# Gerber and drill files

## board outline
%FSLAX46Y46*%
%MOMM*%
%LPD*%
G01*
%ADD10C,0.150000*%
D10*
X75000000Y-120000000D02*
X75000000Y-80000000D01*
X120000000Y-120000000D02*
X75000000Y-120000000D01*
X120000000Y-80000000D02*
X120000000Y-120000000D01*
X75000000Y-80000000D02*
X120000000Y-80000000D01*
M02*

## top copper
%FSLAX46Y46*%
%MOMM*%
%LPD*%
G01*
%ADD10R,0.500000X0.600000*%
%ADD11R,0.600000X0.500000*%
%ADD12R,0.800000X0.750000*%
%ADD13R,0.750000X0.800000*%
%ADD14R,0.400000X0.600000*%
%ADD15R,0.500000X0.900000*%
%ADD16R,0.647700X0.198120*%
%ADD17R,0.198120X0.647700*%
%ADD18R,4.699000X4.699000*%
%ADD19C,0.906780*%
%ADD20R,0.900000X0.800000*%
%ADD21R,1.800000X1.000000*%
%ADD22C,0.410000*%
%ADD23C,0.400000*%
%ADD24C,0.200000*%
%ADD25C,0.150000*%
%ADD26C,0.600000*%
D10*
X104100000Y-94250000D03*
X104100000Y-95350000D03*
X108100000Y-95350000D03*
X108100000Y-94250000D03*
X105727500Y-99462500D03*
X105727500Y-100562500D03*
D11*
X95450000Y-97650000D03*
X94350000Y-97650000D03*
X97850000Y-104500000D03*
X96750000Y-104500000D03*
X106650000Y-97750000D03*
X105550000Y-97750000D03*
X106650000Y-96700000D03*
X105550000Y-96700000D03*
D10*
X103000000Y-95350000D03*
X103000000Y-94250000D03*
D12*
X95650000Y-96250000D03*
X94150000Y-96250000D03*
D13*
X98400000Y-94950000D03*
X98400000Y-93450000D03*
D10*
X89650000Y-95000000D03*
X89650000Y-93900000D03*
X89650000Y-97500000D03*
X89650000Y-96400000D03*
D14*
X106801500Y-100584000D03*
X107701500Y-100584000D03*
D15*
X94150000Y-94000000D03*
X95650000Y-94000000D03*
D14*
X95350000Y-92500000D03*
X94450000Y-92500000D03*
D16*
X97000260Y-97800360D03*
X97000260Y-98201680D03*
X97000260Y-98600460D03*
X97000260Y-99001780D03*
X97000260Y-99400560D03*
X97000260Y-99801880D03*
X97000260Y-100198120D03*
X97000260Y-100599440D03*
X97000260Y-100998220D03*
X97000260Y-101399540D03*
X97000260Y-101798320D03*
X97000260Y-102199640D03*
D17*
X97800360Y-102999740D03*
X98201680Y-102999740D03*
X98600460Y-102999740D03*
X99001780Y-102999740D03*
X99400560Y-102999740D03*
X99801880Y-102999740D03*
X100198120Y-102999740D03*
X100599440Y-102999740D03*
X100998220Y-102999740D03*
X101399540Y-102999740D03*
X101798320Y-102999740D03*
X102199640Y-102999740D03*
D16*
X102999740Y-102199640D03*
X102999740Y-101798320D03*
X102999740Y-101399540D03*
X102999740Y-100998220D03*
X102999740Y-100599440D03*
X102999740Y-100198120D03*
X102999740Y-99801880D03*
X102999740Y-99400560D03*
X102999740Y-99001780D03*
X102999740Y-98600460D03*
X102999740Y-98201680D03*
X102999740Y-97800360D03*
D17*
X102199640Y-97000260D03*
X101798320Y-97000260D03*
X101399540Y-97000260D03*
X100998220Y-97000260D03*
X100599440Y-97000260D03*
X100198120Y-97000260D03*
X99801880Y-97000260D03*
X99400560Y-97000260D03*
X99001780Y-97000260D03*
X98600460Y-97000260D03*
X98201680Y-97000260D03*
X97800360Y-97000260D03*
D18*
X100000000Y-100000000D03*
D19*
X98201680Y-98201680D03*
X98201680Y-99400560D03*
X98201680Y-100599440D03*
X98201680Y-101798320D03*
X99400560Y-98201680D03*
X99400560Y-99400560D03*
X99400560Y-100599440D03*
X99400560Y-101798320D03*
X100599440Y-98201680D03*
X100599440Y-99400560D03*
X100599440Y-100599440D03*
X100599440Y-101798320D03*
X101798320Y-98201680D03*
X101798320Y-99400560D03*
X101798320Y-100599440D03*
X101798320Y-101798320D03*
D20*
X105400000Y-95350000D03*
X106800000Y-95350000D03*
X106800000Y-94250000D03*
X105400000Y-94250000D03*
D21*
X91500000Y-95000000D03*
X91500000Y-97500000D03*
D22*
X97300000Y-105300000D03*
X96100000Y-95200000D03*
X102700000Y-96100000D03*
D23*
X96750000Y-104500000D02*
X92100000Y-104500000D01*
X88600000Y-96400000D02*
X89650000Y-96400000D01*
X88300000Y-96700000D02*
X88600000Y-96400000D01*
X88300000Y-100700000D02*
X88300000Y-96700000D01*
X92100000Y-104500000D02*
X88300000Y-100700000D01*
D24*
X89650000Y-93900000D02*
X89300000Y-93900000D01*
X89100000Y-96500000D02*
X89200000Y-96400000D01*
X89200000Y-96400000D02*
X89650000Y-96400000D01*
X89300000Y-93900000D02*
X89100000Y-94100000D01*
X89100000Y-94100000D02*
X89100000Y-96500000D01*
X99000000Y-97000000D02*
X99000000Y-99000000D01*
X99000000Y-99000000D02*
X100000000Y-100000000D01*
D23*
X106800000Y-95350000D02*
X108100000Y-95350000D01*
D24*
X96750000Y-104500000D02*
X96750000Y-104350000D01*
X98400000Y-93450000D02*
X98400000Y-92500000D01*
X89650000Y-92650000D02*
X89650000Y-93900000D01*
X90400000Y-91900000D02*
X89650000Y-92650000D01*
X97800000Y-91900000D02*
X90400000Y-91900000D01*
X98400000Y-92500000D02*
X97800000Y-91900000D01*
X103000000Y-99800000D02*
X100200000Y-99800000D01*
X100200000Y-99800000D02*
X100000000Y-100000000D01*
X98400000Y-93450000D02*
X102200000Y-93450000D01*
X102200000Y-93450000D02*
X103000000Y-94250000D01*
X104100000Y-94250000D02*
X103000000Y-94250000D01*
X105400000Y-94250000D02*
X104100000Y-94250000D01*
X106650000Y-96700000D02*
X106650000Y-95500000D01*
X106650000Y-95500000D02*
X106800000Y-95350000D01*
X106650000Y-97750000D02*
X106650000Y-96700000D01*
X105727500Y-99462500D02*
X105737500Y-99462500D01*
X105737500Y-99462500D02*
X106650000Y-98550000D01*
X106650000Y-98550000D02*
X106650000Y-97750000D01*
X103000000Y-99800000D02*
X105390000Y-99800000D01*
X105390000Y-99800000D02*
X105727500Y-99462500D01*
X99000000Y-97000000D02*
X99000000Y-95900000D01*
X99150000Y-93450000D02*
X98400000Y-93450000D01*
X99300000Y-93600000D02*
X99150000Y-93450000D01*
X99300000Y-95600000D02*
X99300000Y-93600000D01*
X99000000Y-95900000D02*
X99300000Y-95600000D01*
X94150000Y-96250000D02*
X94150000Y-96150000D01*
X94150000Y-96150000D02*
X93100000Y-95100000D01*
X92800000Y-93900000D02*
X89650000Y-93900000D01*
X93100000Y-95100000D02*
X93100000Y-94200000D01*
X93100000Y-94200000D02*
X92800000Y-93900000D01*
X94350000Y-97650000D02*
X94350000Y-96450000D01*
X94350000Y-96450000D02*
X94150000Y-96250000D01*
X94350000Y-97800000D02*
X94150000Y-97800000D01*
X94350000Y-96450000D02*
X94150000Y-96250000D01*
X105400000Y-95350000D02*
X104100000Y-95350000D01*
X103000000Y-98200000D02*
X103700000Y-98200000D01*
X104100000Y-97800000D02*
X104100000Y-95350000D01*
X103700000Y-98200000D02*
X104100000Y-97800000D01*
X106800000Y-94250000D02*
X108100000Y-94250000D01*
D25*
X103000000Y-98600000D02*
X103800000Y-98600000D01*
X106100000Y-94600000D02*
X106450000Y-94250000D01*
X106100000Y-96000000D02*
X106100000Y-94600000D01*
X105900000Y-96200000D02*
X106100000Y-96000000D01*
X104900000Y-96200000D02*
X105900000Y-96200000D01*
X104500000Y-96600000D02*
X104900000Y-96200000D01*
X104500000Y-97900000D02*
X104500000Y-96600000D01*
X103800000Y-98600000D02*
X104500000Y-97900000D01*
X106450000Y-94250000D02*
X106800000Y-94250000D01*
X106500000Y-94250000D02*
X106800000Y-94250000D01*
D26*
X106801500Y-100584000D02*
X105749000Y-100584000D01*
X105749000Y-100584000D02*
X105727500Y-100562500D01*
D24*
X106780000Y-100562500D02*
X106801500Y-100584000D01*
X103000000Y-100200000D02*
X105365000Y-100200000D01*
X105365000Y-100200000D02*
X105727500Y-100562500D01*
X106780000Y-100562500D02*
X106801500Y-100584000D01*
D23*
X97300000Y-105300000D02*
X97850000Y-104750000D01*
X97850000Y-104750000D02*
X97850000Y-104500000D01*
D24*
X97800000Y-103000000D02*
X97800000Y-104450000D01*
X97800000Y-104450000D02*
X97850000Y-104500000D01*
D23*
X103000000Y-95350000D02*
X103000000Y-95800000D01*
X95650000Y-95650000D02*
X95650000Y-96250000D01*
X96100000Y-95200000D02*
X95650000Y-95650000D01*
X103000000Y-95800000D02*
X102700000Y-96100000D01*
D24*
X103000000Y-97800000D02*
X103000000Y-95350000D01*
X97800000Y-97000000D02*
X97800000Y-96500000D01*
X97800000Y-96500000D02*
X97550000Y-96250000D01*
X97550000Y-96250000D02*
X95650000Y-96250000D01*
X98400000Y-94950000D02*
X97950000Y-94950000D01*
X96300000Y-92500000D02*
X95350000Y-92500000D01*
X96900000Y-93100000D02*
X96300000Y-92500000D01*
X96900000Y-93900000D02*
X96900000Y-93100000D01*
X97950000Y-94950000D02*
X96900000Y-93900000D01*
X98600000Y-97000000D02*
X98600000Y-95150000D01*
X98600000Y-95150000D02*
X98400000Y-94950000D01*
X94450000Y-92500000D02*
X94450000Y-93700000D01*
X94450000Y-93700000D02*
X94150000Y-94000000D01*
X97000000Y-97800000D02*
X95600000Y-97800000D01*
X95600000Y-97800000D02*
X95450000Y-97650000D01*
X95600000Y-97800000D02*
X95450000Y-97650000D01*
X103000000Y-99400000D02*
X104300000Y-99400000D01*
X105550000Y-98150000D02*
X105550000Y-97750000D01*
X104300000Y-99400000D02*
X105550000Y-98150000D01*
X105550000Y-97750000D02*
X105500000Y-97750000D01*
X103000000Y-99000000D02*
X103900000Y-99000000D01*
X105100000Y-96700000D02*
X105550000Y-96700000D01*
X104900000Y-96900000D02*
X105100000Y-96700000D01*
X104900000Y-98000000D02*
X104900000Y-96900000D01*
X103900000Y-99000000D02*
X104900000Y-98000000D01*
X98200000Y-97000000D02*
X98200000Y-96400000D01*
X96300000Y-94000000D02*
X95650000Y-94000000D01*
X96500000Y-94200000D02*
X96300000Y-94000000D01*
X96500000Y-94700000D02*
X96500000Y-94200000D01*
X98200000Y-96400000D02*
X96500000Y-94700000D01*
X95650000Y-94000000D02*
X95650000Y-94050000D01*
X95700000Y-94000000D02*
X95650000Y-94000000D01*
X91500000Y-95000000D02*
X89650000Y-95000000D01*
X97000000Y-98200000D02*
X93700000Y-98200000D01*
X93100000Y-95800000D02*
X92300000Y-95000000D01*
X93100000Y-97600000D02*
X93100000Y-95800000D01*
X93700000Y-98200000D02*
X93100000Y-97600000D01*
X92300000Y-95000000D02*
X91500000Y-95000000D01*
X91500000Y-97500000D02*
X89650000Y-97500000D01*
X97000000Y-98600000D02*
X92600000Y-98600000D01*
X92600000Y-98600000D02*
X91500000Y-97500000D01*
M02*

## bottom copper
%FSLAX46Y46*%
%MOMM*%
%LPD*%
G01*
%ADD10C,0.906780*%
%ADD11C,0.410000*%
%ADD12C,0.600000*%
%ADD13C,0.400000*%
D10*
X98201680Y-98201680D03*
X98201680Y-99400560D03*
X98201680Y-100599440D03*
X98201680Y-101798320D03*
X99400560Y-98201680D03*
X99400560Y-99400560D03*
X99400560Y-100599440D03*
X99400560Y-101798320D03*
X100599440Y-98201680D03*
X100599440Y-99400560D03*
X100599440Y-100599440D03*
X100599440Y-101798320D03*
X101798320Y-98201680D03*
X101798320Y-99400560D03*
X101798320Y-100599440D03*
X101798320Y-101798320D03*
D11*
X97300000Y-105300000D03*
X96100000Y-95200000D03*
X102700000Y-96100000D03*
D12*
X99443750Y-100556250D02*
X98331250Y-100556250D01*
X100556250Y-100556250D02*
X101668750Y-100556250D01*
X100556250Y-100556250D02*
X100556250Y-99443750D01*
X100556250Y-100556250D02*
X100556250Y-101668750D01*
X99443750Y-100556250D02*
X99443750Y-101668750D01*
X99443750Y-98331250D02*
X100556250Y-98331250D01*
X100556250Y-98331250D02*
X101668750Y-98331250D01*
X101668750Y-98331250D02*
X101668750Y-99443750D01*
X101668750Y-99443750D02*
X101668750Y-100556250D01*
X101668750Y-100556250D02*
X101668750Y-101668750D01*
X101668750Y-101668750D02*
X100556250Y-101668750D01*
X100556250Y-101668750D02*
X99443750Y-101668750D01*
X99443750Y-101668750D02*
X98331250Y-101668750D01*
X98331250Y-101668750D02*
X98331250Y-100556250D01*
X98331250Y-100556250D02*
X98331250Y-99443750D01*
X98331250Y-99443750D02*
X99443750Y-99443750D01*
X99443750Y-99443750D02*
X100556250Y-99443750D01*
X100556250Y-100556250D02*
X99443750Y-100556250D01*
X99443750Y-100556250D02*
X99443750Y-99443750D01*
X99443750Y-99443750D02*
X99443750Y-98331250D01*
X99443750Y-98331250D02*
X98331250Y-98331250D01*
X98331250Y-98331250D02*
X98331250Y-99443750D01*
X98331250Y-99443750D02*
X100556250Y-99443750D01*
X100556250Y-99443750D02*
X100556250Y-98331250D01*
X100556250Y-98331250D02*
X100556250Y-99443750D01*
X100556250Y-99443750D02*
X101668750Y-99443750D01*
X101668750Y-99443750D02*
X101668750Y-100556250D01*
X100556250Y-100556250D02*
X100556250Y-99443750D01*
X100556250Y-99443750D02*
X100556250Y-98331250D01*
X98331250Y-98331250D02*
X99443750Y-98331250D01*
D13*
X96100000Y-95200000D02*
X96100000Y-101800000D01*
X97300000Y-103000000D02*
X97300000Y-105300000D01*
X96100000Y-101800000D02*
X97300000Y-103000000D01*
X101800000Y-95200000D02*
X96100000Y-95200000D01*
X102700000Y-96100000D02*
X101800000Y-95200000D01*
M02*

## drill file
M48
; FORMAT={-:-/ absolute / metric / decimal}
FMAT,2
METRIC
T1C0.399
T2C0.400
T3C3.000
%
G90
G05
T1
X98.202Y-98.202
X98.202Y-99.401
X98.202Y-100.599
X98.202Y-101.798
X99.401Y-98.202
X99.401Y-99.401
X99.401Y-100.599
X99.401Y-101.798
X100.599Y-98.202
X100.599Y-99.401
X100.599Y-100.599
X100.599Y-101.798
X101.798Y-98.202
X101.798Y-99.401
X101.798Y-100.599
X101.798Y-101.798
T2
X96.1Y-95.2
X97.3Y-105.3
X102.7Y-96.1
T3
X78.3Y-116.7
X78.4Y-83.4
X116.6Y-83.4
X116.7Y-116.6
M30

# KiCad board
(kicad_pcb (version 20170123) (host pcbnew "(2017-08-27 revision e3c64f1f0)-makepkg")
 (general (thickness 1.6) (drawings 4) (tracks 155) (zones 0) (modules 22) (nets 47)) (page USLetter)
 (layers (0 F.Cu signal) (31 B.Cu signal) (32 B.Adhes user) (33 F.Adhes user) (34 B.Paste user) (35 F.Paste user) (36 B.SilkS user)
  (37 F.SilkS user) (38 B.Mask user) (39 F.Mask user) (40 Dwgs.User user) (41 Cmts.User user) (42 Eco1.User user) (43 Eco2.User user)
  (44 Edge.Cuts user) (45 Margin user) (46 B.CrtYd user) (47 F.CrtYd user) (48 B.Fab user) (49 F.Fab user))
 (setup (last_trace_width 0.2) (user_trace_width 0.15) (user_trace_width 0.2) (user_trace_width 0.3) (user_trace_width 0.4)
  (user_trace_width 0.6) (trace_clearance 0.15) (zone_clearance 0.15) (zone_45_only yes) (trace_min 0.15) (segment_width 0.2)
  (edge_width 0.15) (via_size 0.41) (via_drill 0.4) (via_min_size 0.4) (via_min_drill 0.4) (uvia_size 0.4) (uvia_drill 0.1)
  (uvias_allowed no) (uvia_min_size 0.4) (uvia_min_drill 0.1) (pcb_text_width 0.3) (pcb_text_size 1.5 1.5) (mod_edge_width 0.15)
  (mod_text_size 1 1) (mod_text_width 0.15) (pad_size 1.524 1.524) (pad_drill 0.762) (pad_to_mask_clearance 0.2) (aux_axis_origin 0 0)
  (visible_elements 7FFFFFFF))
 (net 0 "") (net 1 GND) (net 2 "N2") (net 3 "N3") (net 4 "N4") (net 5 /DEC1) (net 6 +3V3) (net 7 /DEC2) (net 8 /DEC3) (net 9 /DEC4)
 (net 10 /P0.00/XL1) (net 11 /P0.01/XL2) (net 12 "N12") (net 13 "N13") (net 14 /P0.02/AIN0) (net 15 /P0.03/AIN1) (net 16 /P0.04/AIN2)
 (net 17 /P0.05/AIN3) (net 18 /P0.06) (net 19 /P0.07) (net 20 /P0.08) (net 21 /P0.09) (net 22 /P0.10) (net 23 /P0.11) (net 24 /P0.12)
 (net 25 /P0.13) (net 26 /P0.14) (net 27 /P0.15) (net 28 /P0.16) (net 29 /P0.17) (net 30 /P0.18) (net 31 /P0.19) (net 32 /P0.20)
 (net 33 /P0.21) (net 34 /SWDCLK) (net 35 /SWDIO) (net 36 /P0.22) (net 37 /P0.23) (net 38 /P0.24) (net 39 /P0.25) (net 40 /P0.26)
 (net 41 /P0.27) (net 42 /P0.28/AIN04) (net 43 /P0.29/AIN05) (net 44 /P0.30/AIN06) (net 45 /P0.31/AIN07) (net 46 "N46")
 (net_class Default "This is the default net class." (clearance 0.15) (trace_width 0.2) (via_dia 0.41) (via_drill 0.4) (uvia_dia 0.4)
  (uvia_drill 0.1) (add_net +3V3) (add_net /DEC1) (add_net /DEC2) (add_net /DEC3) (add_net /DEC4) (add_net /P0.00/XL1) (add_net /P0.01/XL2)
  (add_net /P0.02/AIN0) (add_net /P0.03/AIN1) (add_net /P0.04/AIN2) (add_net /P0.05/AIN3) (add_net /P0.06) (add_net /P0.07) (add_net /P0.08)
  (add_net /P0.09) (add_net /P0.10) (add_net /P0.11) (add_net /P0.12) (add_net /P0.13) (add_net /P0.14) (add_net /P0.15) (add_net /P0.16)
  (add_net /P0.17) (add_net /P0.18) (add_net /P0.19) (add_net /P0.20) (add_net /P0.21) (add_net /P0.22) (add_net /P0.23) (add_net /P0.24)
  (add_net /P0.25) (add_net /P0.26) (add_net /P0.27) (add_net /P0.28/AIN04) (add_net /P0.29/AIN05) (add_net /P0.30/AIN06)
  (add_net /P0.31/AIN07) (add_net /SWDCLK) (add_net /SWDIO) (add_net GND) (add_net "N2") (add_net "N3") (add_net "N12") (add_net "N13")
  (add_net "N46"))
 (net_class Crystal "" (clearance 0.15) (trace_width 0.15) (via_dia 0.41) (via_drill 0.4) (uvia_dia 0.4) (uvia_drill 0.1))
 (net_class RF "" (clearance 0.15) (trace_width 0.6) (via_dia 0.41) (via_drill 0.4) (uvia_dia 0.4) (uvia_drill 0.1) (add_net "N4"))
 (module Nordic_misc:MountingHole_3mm (layer F.Cu) (at 78.3 116.7)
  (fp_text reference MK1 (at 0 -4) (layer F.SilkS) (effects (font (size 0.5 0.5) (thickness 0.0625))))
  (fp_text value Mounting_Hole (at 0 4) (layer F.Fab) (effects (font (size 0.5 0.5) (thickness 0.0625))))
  (pad 1 np_thru_hole circle (at 0 0) (size 3 3) (drill 3) (layers *.Cu *.Mask)))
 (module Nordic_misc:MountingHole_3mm (layer F.Cu) (at 116.7 116.6)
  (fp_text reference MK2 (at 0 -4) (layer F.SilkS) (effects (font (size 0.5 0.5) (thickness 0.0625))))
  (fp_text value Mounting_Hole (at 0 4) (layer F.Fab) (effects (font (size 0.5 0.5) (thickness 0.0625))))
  (pad 1 np_thru_hole circle (at 0 0) (size 3 3) (drill 3) (layers *.Cu *.Mask)))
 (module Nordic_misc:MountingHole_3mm (layer F.Cu) (at 116.6 83.4)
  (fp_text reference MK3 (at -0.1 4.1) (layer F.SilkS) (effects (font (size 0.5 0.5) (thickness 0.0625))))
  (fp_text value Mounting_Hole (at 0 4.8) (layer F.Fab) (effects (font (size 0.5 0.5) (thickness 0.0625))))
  (pad 1 np_thru_hole circle (at 0 0) (size 3 3) (drill 3) (layers *.Cu *.Mask)))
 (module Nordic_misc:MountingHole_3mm (layer F.Cu) (at 78.4 83.4)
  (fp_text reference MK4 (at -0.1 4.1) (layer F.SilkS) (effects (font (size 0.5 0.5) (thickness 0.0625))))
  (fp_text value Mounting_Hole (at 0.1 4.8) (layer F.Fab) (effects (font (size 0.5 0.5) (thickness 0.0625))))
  (pad 1 np_thru_hole circle (at 0 0) (size 3 3) (drill 3) (layers *.Cu *.Mask)))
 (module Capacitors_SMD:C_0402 (layer F.Cu) (at 104.1 94.8 270)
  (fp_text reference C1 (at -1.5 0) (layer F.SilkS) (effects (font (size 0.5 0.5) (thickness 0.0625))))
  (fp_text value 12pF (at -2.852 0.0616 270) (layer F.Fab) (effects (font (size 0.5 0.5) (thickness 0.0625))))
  (pad 1 smd rect (at -0.55 0 270) (size 0.6 0.5) (layers F.Cu F.Paste F.Mask) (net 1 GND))
  (pad 2 smd rect (at 0.55 0 270) (size 0.6 0.5) (layers F.Cu F.Paste F.Mask) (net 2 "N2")))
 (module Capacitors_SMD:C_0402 (layer F.Cu) (at 108.1 94.8 90)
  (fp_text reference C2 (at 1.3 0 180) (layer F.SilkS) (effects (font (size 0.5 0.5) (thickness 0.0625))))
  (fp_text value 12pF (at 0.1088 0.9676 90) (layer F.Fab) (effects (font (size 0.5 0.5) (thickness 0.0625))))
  (pad 1 smd rect (at -0.55 0 90) (size 0.6 0.5) (layers F.Cu F.Paste F.Mask) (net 1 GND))
  (pad 2 smd rect (at 0.55 0 90) (size 0.6 0.5) (layers F.Cu F.Paste F.Mask) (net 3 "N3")))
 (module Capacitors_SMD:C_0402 (layer F.Cu) (at 105.7275 100.0125 270)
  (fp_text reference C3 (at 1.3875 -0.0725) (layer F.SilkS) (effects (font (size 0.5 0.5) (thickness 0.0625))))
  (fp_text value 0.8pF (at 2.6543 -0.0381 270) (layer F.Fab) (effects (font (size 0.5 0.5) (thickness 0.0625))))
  (pad 1 smd rect (at -0.55 0 270) (size 0.6 0.5) (layers F.Cu F.Paste F.Mask) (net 1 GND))
  (pad 2 smd rect (at 0.55 0 270) (size 0.6 0.5) (layers F.Cu F.Paste F.Mask) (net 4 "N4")))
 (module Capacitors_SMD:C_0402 (layer F.Cu) (at 94.9 97.65 180)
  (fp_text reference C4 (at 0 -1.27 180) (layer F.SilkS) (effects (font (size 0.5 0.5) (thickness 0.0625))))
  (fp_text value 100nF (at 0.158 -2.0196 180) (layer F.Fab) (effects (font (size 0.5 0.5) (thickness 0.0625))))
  (pad 1 smd rect (at -0.55 0 180) (size 0.6 0.5) (layers F.Cu F.Paste F.Mask) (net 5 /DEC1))
  (pad 2 smd rect (at 0.55 0 180) (size 0.6 0.5) (layers F.Cu F.Paste F.Mask) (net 1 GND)))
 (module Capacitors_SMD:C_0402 (layer F.Cu) (at 97.3 104.5 180)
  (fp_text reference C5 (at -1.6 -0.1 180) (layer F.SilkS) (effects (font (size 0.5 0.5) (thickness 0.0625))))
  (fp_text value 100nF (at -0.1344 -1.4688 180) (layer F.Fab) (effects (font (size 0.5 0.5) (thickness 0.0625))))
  (pad 1 smd rect (at -0.55 0 180) (size 0.6 0.5) (layers F.Cu F.Paste F.Mask) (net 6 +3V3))
  (pad 2 smd rect (at 0.55 0 180) (size 0.6 0.5) (layers F.Cu F.Paste F.Mask) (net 1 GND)))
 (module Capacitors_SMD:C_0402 (layer F.Cu) (at 106.1 97.75 180)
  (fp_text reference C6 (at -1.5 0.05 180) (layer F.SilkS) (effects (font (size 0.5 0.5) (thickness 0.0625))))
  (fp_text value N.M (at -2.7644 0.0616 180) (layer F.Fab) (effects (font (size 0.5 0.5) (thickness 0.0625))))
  (pad 1 smd rect (at -0.55 0 180) (size 0.6 0.5) (layers F.Cu F.Paste F.Mask) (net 1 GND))
  (pad 2 smd rect (at 0.55 0 180) (size 0.6 0.5) (layers F.Cu F.Paste F.Mask) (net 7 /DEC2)))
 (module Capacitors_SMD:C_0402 (layer F.Cu) (at 106.1 96.7 180)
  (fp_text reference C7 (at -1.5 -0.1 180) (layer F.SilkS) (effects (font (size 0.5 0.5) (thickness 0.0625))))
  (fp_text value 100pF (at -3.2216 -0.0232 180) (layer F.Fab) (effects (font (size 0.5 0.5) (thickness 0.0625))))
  (pad 1 smd rect (at -0.55 0 180) (size 0.6 0.5) (layers F.Cu F.Paste F.Mask) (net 1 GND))
  (pad 2 smd rect (at 0.55 0 180) (size 0.6 0.5) (layers F.Cu F.Paste F.Mask) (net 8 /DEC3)))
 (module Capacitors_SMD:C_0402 (layer F.Cu) (at 103 94.8 90)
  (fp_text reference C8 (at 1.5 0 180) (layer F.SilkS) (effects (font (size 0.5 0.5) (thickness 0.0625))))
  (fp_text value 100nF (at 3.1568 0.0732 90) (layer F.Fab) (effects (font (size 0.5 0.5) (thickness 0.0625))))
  (pad 1 smd rect (at -0.55 0 90) (size 0.6 0.5) (layers F.Cu F.Paste F.Mask) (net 6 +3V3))
  (pad 2 smd rect (at 0.55 0 90) (size 0.6 0.5) (layers F.Cu F.Paste F.Mask) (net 1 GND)))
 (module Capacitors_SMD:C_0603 (layer F.Cu) (at 94.9 96.25 180)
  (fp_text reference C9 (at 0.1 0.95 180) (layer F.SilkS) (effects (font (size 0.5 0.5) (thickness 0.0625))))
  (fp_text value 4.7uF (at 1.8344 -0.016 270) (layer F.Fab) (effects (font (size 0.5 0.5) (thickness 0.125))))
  (pad 1 smd rect (at -0.75 0 180) (size 0.8 0.75) (layers F.Cu F.Paste F.Mask) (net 6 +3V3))
  (pad 2 smd rect (at 0.75 0 180) (size 0.8 0.75) (layers F.Cu F.Paste F.Mask) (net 1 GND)))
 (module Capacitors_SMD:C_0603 (layer F.Cu) (at 98.4 94.2 90)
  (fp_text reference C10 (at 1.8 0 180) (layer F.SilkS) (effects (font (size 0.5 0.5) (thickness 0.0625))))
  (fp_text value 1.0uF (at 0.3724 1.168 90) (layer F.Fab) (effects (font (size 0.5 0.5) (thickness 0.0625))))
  (pad 1 smd rect (at -0.75 0 90) (size 0.8 0.75) (layers F.Cu F.Paste F.Mask) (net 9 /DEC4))
  (pad 2 smd rect (at 0.75 0 90) (size 0.8 0.75) (layers F.Cu F.Paste F.Mask) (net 1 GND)))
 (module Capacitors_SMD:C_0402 (layer F.Cu) (at 89.65 94.45 90)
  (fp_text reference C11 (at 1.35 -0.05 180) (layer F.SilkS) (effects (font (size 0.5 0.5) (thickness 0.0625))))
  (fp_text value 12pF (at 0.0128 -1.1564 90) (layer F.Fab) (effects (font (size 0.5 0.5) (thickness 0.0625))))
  (pad 1 smd rect (at -0.55 0 90) (size 0.6 0.5) (layers F.Cu F.Paste F.Mask) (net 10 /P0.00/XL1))
  (pad 2 smd rect (at 0.55 0 90) (size 0.6 0.5) (layers F.Cu F.Paste F.Mask) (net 1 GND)))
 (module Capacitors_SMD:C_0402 (layer F.Cu) (at 89.65 96.95 90)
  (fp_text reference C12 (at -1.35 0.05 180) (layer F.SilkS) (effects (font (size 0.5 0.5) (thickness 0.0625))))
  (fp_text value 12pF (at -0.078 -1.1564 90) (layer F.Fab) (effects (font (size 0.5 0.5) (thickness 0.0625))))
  (pad 1 smd rect (at -0.55 0 90) (size 0.6 0.5) (layers F.Cu F.Paste F.Mask) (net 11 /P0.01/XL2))
  (pad 2 smd rect (at 0.55 0 90) (size 0.6 0.5) (layers F.Cu F.Paste F.Mask) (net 1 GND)))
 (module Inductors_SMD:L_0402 (layer F.Cu) (at 107.2515 100.584)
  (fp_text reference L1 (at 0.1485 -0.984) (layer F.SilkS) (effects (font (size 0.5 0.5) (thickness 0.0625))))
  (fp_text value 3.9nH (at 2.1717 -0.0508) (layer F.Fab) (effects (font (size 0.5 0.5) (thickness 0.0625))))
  (pad 1 smd rect (at -0.45 0) (size 0.4 0.6) (layers F.Cu F.Paste F.Mask) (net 4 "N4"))
  (pad 2 smd rect (at 0.45 0) (size 0.4 0.6) (layers F.Cu F.Paste F.Mask)))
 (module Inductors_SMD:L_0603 (layer F.Cu) (at 94.9 94)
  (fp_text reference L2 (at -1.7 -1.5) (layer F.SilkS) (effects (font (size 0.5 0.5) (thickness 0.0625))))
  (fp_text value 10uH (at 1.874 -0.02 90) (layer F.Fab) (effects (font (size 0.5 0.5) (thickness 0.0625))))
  (pad 1 smd rect (at -0.75 0) (size 0.5 0.9) (layers F.Cu F.Paste F.Mask) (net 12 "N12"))
  (pad 2 smd rect (at 0.75 0) (size 0.5 0.9) (layers F.Cu F.Paste F.Mask) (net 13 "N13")))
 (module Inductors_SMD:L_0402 (layer F.Cu) (at 94.9 92.5 180)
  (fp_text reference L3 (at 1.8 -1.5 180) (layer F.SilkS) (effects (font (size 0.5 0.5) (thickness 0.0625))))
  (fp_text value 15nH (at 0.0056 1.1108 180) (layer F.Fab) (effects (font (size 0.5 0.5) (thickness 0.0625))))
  (pad 1 smd rect (at -0.45 0 180) (size 0.4 0.6) (layers F.Cu F.Paste F.Mask) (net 9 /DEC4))
  (pad 2 smd rect (at 0.45 0 180) (size 0.4 0.6) (layers F.Cu F.Paste F.Mask) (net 12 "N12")))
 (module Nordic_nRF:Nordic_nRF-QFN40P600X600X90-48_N (layer F.Cu) (at 100 100)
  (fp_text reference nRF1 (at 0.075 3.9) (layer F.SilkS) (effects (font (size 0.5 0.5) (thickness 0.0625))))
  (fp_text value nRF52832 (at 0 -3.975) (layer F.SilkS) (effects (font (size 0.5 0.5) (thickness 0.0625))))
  (pad 1 smd rect (at -2.99974 -2.19964) (size 0.6477 0.19812) (layers F.Cu F.Paste F.Mask) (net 5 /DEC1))
  (pad 2 smd rect (at -2.99974 -1.79832) (size 0.6477 0.19812) (layers F.Cu F.Paste F.Mask) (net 10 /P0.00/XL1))
  (pad 3 smd rect (at -2.99974 -1.39954) (size 0.6477 0.19812) (layers F.Cu F.Paste F.Mask) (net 11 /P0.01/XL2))
  (pad 4 smd rect (at -2.99974 -0.99822) (size 0.6477 0.19812) (layers F.Cu F.Paste F.Mask) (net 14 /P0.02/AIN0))
  (pad 5 smd rect (at -2.99974 -0.59944) (size 0.6477 0.19812) (layers F.Cu F.Paste F.Mask) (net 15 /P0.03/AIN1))
  (pad 6 smd rect (at -2.99974 -0.19812) (size 0.6477 0.19812) (layers F.Cu F.Paste F.Mask) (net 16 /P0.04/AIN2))
  (pad 7 smd rect (at -2.99974 0.19812) (size 0.6477 0.19812) (layers F.Cu F.Paste F.Mask) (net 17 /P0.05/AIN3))
  (pad 8 smd rect (at -2.99974 0.59944) (size 0.6477 0.19812) (layers F.Cu F.Paste F.Mask) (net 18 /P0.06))
  (pad 9 smd rect (at -2.99974 0.99822) (size 0.6477 0.19812) (layers F.Cu F.Paste F.Mask) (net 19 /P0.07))
  (pad 10 smd rect (at -2.99974 1.39954) (size 0.6477 0.19812) (layers F.Cu F.Paste F.Mask) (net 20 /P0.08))
  (pad 11 smd rect (at -2.99974 1.79832) (size 0.6477 0.19812) (layers F.Cu F.Paste F.Mask) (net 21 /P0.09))
  (pad 12 smd rect (at -2.99974 2.19964) (size 0.6477 0.19812) (layers F.Cu F.Paste F.Mask) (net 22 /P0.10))
  (pad 13 smd rect (at -2.19964 2.99974 90) (size 0.6477 0.19812) (layers F.Cu F.Paste F.Mask) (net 6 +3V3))
  (pad 14 smd rect (at -1.79832 2.99974 90) (size 0.6477 0.19812) (layers F.Cu F.Paste F.Mask) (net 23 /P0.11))
  (pad 15 smd rect (at -1.39954 2.99974 90) (size 0.6477 0.19812) (layers F.Cu F.Paste F.Mask) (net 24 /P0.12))
  (pad 16 smd rect (at -0.99822 2.99974 90) (size 0.6477 0.19812) (layers F.Cu F.Paste F.Mask) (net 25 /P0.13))
  (pad 17 smd rect (at -0.59944 2.99974 90) (size 0.6477 0.19812) (layers F.Cu F.Paste F.Mask) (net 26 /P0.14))
  (pad 18 smd rect (at -0.19812 2.99974 90) (size 0.6477 0.19812) (layers F.Cu F.Paste F.Mask) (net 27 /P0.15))
  (pad 19 smd rect (at 0.19812 2.99974 90) (size 0.6477 0.19812) (layers F.Cu F.Paste F.Mask) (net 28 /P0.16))
  (pad 20 smd rect (at 0.59944 2.99974 90) (size 0.6477 0.19812) (layers F.Cu F.Paste F.Mask) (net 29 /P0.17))
  (pad 21 smd rect (at 0.99822 2.99974 90) (size 0.6477 0.19812) (layers F.Cu F.Paste F.Mask) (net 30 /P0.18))
  (pad 22 smd rect (at 1.39954 2.99974 90) (size 0.6477 0.19812) (layers F.Cu F.Paste F.Mask) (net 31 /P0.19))
  (pad 23 smd rect (at 1.79832 2.99974 90) (size 0.6477 0.19812) (layers F.Cu F.Paste F.Mask) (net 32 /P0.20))
  (pad 24 smd rect (at 2.19964 2.99974 90) (size 0.6477 0.19812) (layers F.Cu F.Paste F.Mask) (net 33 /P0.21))
  (pad 25 smd rect (at 2.99974 2.19964 180) (size 0.6477 0.19812) (layers F.Cu F.Paste F.Mask) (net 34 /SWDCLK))
  (pad 26 smd rect (at 2.99974 1.79832 180) (size 0.6477 0.19812) (layers F.Cu F.Paste F.Mask) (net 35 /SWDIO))
  (pad 27 smd rect (at 2.99974 1.39954 180) (size 0.6477 0.19812) (layers F.Cu F.Paste F.Mask) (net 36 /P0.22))
  (pad 28 smd rect (at 2.99974 0.99822 180) (size 0.6477 0.19812) (layers F.Cu F.Paste F.Mask) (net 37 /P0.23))
  (pad 29 smd rect (at 2.99974 0.59944 180) (size 0.6477 0.19812) (layers F.Cu F.Paste F.Mask) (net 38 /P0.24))
  (pad 30 smd rect (at 2.99974 0.19812 180) (size 0.6477 0.19812) (layers F.Cu F.Paste F.Mask) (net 4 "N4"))
  (pad 31 smd rect (at 2.99974 -0.19812 180) (size 0.6477 0.19812) (layers F.Cu F.Paste F.Mask) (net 1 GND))
  (pad 32 smd rect (at 2.99974 -0.59944 180) (size 0.6477 0.19812) (layers F.Cu F.Paste F.Mask) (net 7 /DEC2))
  (pad 33 smd rect (at 2.99974 -0.99822 180) (size 0.6477 0.19812) (layers F.Cu F.Paste F.Mask) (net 8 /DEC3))
  (pad 34 smd rect (at 2.99974 -1.39954 180) (size 0.6477 0.19812) (layers F.Cu F.Paste F.Mask) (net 3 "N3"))
  (pad 35 smd rect (at 2.99974 -1.79832 180) (size 0.6477 0.19812) (layers F.Cu F.Paste F.Mask) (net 2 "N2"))
  (pad 36 smd rect (at 2.99974 -2.19964 180) (size 0.6477 0.19812) (layers F.Cu F.Paste F.Mask) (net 6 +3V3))
  (pad 37 smd rect (at 2.19964 -2.99974 270) (size 0.6477 0.19812) (layers F.Cu F.Paste F.Mask) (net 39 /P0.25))
  (pad 38 smd rect (at 1.79832 -2.99974 270) (size 0.6477 0.19812) (layers F.Cu F.Paste F.Mask) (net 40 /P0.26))
  (pad 39 smd rect (at 1.39954 -2.99974 270) (size 0.6477 0.19812) (layers F.Cu F.Paste F.Mask) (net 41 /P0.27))
  (pad 40 smd rect (at 0.99822 -2.99974 270) (size 0.6477 0.19812) (layers F.Cu F.Paste F.Mask) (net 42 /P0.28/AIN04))
  (pad 41 smd rect (at 0.59944 -2.99974 270) (size 0.6477 0.19812) (layers F.Cu F.Paste F.Mask) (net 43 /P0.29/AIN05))
  (pad 42 smd rect (at 0.19812 -2.99974 270) (size 0.6477 0.19812) (layers F.Cu F.Paste F.Mask) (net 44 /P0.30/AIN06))
  (pad 43 smd rect (at -0.19812 -2.99974 270) (size 0.6477 0.19812) (layers F.Cu F.Paste F.Mask) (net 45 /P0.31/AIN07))
  (pad 44 smd rect (at -0.59944 -2.99974 270) (size 0.6477 0.19812) (layers F.Cu F.Paste F.Mask) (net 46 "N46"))
  (pad 45 smd rect (at -0.99822 -2.99974 270) (size 0.6477 0.19812) (layers F.Cu F.Paste F.Mask) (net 1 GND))
  (pad 46 smd rect (at -1.39954 -2.99974 270) (size 0.6477 0.19812) (layers F.Cu F.Paste F.Mask) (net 9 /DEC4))
  (pad 47 smd rect (at -1.79832 -2.99974 270) (size 0.6477 0.19812) (layers F.Cu F.Paste F.Mask) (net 13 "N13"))
  (pad 48 smd rect (at -2.19964 -2.99974 270) (size 0.6477 0.19812) (layers F.Cu F.Paste F.Mask) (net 6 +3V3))
  (pad 49 smd rect (at 0 0) (size 4.699 4.699) (layers F.Cu F.Paste F.Mask) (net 1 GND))
  (pad 49 thru_hole circle (at -1.79832 -1.79832 270) (size 0.90678 0.90678) (drill 0.39878) (layers *.Cu B.Mask) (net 1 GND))
  (pad 49 thru_hole circle (at -1.79832 -0.59944 270) (size 0.90678 0.90678) (drill 0.39878) (layers *.Cu B.Mask) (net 1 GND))
  (pad 49 thru_hole circle (at -1.79832 0.59944 270) (size 0.90678 0.90678) (drill 0.39878) (layers *.Cu B.Mask) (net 1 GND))
  (pad 49 thru_hole circle (at -1.79832 1.79832 270) (size 0.90678 0.90678) (drill 0.39878) (layers *.Cu B.Mask) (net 1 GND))
  (pad 49 thru_hole circle (at -0.59944 -1.79832 270) (size 0.90678 0.90678) (drill 0.39878) (layers *.Cu B.Mask) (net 1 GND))
  (pad 49 thru_hole circle (at -0.59944 -0.59944 270) (size 0.90678 0.90678) (drill 0.39878) (layers *.Cu B.Mask) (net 1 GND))
  (pad 49 thru_hole circle (at -0.59944 0.59944 270) (size 0.90678 0.90678) (drill 0.39878) (layers *.Cu B.Mask) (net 1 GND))
  (pad 49 thru_hole circle (at -0.59944 1.79832 270) (size 0.90678 0.90678) (drill 0.39878) (layers *.Cu B.Mask) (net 1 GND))
  (pad 49 thru_hole circle (at 0.59944 -1.79832 270) (size 0.90678 0.90678) (drill 0.39878) (layers *.Cu B.Mask) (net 1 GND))
  (pad 49 thru_hole circle (at 0.59944 -0.59944 270) (size 0.90678 0.90678) (drill 0.39878) (layers *.Cu B.Mask) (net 1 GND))
  (pad 49 thru_hole circle (at 0.59944 0.59944 270) (size 0.90678 0.90678) (drill 0.39878) (layers *.Cu B.Mask) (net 1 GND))
  (pad 49 thru_hole circle (at 0.59944 1.79832 270) (size 0.90678 0.90678) (drill 0.39878) (layers *.Cu B.Mask) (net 1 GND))
  (pad 49 thru_hole circle (at 1.79832 -1.79832 270) (size 0.90678 0.90678) (drill 0.39878) (layers *.Cu B.Mask) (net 1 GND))
  (pad 49 thru_hole circle (at 1.79832 -0.59944 270) (size 0.90678 0.90678) (drill 0.39878) (layers *.Cu B.Mask) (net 1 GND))
  (pad 49 thru_hole circle (at 1.79832 0.59944 270) (size 0.90678 0.90678) (drill 0.39878) (layers *.Cu B.Mask) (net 1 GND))
  (pad 49 thru_hole circle (at 1.79832 1.79832 270) (size 0.90678 0.90678) (drill 0.39878) (layers *.Cu B.Mask) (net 1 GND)))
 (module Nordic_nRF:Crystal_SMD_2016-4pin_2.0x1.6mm (layer F.Cu) (at 106.1 94.8)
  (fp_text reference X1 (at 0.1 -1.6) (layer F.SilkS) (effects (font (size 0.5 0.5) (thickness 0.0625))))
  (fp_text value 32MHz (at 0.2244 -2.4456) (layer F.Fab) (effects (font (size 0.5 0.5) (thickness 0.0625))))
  (pad 1 smd rect (at -0.7 0.55) (size 0.9 0.8) (layers F.Cu F.Paste F.Mask) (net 2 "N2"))
  (pad 2 smd rect (at 0.7 0.55) (size 0.9 0.8) (layers F.Cu F.Paste F.Mask) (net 1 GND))
  (pad 3 smd rect (at 0.7 -0.55) (size 0.9 0.8) (layers F.Cu F.Paste F.Mask) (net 3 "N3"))
  (pad 4 smd rect (at -0.7 -0.55) (size 0.9 0.8) (layers F.Cu F.Paste F.Mask) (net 1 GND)))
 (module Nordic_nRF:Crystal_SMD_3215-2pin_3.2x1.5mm (layer F.Cu) (at 91.5 96.25 90)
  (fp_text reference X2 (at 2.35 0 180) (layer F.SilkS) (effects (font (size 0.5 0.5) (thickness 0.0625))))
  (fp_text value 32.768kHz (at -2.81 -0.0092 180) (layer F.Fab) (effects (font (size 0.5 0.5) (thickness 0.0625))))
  (pad 1 smd rect (at 1.25 0 90) (size 1 1.8) (layers F.Cu F.Paste F.Mask) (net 10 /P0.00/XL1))
  (pad 2 smd rect (at -1.25 0 90) (size 1 1.8) (layers F.Cu F.Paste F.Mask) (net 11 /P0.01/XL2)))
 (gr_line (start 75 120) (end 75 80) (angle 90) (layer Edge.Cuts) (width 0.15))
 (gr_line (start 120 120) (end 75 120) (angle 90) (layer Edge.Cuts) (width 0.15))
 (gr_line (start 120 80) (end 120 120) (angle 90) (layer Edge.Cuts) (width 0.15))
 (gr_line (start 75 80) (end 120 80) (angle 90) (layer Edge.Cuts) (width 0.15))
 (segment (start 96.75 104.5) (end 92.1 104.5) (width 0.4) (layer F.Cu) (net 1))
 (segment (start 88.6 96.4) (end 89.65 96.4) (width 0.4) (layer F.Cu) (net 1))
 (segment (start 88.3 96.7) (end 88.6 96.4) (width 0.4) (layer F.Cu) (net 1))
 (segment (start 88.3 100.7) (end 88.3 96.7) (width 0.4) (layer F.Cu) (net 1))
 (segment (start 92.1 104.5) (end 88.3 100.7) (width 0.4) (layer F.Cu) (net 1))
 (segment (start 89.65 93.9) (end 89.3 93.9) (width 0.2) (layer F.Cu) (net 1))
 (segment (start 89.1 96.5) (end 89.2 96.4) (width 0.2) (layer F.Cu) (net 1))
 (segment (start 89.2 96.4) (end 89.65 96.4) (width 0.2) (layer F.Cu) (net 1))
 (segment (start 89.3 93.9) (end 89.1 94.1) (width 0.2) (layer F.Cu) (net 1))
 (segment (start 89.1 94.1) (end 89.1 96.5) (width 0.2) (layer F.Cu) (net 1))
 (segment (start 99 97) (end 99 99) (width 0.2) (layer F.Cu) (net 1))
 (segment (start 99 99) (end 100 100) (width 0.2) (layer F.Cu) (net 1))
 (segment (start 106.8 95.35) (end 108.1 95.35) (width 0.4) (layer F.Cu) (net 1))
 (segment (start 96.75 104.5) (end 96.75 104.35) (width 0.2) (layer F.Cu) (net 1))
 (segment (start 98.4 93.45) (end 98.4 92.5) (width 0.2) (layer F.Cu) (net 1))
 (segment (start 89.65 92.65) (end 89.65 93.9) (width 0.2) (layer F.Cu) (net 1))
 (segment (start 90.4 91.9) (end 89.65 92.65) (width 0.2) (layer F.Cu) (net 1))
 (segment (start 97.8 91.9) (end 90.4 91.9) (width 0.2) (layer F.Cu) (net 1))
 (segment (start 98.4 92.5) (end 97.8 91.9) (width 0.2) (layer F.Cu) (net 1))
 (segment (start 99.44375 100.55625) (end 98.33125 100.55625) (width 0.6) (layer B.Cu) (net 1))
 (segment (start 100.55625 100.55625) (end 101.66875 100.55625) (width 0.6) (layer B.Cu) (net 1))
 (segment (start 100.55625 100.55625) (end 100.55625 99.44375) (width 0.6) (layer B.Cu) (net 1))
 (segment (start 100.55625 100.55625) (end 100.55625 101.66875) (width 0.6) (layer B.Cu) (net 1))
 (segment (start 99.44375 100.55625) (end 99.44375 101.66875) (width 0.6) (layer B.Cu) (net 1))
 (segment (start 99.44375 98.33125) (end 100.55625 98.33125) (width 0.6) (layer B.Cu) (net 1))
 (segment (start 100.55625 98.33125) (end 101.66875 98.33125) (width 0.6) (layer B.Cu) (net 1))
 (segment (start 101.66875 98.33125) (end 101.66875 99.44375) (width 0.6) (layer B.Cu) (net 1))
 (segment (start 101.66875 99.44375) (end 101.66875 100.55625) (width 0.6) (layer B.Cu) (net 1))
 (segment (start 101.66875 100.55625) (end 101.66875 101.66875) (width 0.6) (layer B.Cu) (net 1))
 (segment (start 101.66875 101.66875) (end 100.55625 101.66875) (width 0.6) (layer B.Cu) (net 1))
 (segment (start 100.55625 101.66875) (end 99.44375 101.66875) (width 0.6) (layer B.Cu) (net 1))
 (segment (start 99.44375 101.66875) (end 98.33125 101.66875) (width 0.6) (layer B.Cu) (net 1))
 (segment (start 98.33125 101.66875) (end 98.33125 100.55625) (width 0.6) (layer B.Cu) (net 1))
 (segment (start 98.33125 100.55625) (end 98.33125 99.44375) (width 0.6) (layer B.Cu) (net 1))
 (segment (start 98.33125 99.44375) (end 99.44375 99.44375) (width 0.6) (layer B.Cu) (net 1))
 (segment (start 99.44375 99.44375) (end 100.55625 99.44375) (width 0.6) (layer B.Cu) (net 1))
 (segment (start 100.55625 100.55625) (end 99.44375 100.55625) (width 0.6) (layer B.Cu) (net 1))
 (segment (start 99.44375 100.55625) (end 99.44375 99.44375) (width 0.6) (layer B.Cu) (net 1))
 (segment (start 99.44375 99.44375) (end 99.44375 98.33125) (width 0.6) (layer B.Cu) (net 1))
 (segment (start 99.44375 98.33125) (end 98.33125 98.33125) (width 0.6) (layer B.Cu) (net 1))
 (segment (start 98.33125 98.33125) (end 98.33125 99.44375) (width 0.6) (layer B.Cu) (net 1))
 (segment (start 98.33125 99.44375) (end 100.55625 99.44375) (width 0.6) (layer B.Cu) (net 1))
 (segment (start 100.55625 99.44375) (end 100.55625 98.33125) (width 0.6) (layer B.Cu) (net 1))
 (segment (start 100.55625 98.33125) (end 100.55625 99.44375) (width 0.6) (layer B.Cu) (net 1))
 (segment (start 100.55625 99.44375) (end 101.66875 99.44375) (width 0.6) (layer B.Cu) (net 1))
 (segment (start 101.66875 99.44375) (end 101.66875 100.55625) (width 0.6) (layer B.Cu) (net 1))
 (segment (start 100.55625 100.55625) (end 100.55625 99.44375) (width 0.6) (layer B.Cu) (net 1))
 (segment (start 100.55625 99.44375) (end 100.55625 98.33125) (width 0.6) (layer B.Cu) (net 1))
 (segment (start 98.33125 98.33125) (end 99.44375 98.33125) (width 0.6) (layer B.Cu) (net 1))
 (segment (start 103 99.8) (end 100.2 99.8) (width 0.2) (layer F.Cu) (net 1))
 (segment (start 100.2 99.8) (end 100 100) (width 0.2) (layer F.Cu) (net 1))
 (segment (start 98.4 93.45) (end 102.2 93.45) (width 0.2) (layer F.Cu) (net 1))
 (segment (start 102.2 93.45) (end 103 94.25) (width 0.2) (layer F.Cu) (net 1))
 (segment (start 104.1 94.25) (end 103 94.25) (width 0.2) (layer F.Cu) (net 1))
 (segment (start 105.4 94.25) (end 104.1 94.25) (width 0.2) (layer F.Cu) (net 1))
 (segment (start 106.65 96.7) (end 106.65 95.5) (width 0.2) (layer F.Cu) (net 1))
 (segment (start 106.65 95.5) (end 106.8 95.35) (width 0.2) (layer F.Cu) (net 1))
 (segment (start 106.65 97.75) (end 106.65 96.7) (width 0.2) (layer F.Cu) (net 1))
 (segment (start 105.7275 99.4625) (end 105.7375 99.4625) (width 0.2) (layer F.Cu) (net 1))
 (segment (start 105.7375 99.4625) (end 106.65 98.55) (width 0.2) (layer F.Cu) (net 1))
 (segment (start 106.65 98.55) (end 106.65 97.75) (width 0.2) (layer F.Cu) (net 1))
 (segment (start 103 99.8) (end 105.39 99.8) (width 0.2) (layer F.Cu) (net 1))
 (segment (start 105.39 99.8) (end 105.7275 99.4625) (width 0.2) (layer F.Cu) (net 1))
 (segment (start 99 97) (end 99 95.9) (width 0.2) (layer F.Cu) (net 1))
 (segment (start 99.15 93.45) (end 98.4 93.45) (width 0.2) (layer F.Cu) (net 1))
 (segment (start 99.3 93.6) (end 99.15 93.45) (width 0.2) (layer F.Cu) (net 1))
 (segment (start 99.3 95.6) (end 99.3 93.6) (width 0.2) (layer F.Cu) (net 1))
 (segment (start 99 95.9) (end 99.3 95.6) (width 0.2) (layer F.Cu) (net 1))
 (segment (start 94.15 96.25) (end 94.15 96.15) (width 0.2) (layer F.Cu) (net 1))
 (segment (start 94.15 96.15) (end 93.1 95.1) (width 0.2) (layer F.Cu) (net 1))
 (segment (start 92.8 93.9) (end 89.65 93.9) (width 0.2) (layer F.Cu) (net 1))
 (segment (start 93.1 95.1) (end 93.1 94.2) (width 0.2) (layer F.Cu) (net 1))
 (segment (start 93.1 94.2) (end 92.8 93.9) (width 0.2) (layer F.Cu) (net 1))
 (segment (start 94.35 97.65) (end 94.35 96.45) (width 0.2) (layer F.Cu) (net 1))
 (segment (start 94.35 96.45) (end 94.15 96.25) (width 0.2) (layer F.Cu) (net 1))
 (segment (start 94.35 97.8) (end 94.15 97.8) (width 0.2) (layer F.Cu) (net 1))
 (segment (start 94.35 96.45) (end 94.15 96.25) (width 0.2) (layer F.Cu) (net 1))
 (segment (start 105.4 95.35) (end 104.1 95.35) (width 0.2) (layer F.Cu) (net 2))
 (segment (start 103 98.2) (end 103.7 98.2) (width 0.2) (layer F.Cu) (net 2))
 (segment (start 104.1 97.8) (end 104.1 95.35) (width 0.2) (layer F.Cu) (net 2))
 (segment (start 103.7 98.2) (end 104.1 97.8) (width 0.2) (layer F.Cu) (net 2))
 (segment (start 106.8 94.25) (end 108.1 94.25) (width 0.2) (layer F.Cu) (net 3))
 (segment (start 103 98.6) (end 103.8 98.6) (width 0.15) (layer F.Cu) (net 3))
 (segment (start 106.1 94.6) (end 106.45 94.25) (width 0.15) (layer F.Cu) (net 3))
 (segment (start 106.1 96) (end 106.1 94.6) (width 0.15) (layer F.Cu) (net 3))
 (segment (start 105.9 96.2) (end 106.1 96) (width 0.15) (layer F.Cu) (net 3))
 (segment (start 104.9 96.2) (end 105.9 96.2) (width 0.15) (layer F.Cu) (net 3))
 (segment (start 104.5 96.6) (end 104.9 96.2) (width 0.15) (layer F.Cu) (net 3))
 (segment (start 104.5 97.9) (end 104.5 96.6) (width 0.15) (layer F.Cu) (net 3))
 (segment (start 103.8 98.6) (end 104.5 97.9) (width 0.15) (layer F.Cu) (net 3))
 (segment (start 106.45 94.25) (end 106.8 94.25) (width 0.15) (layer F.Cu) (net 3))
 (segment (start 106.5 94.25) (end 106.8 94.25) (width 0.15) (layer F.Cu) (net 3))
 (segment (start 106.8015 100.584) (end 105.749 100.584) (width 0.6) (layer F.Cu) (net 4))
 (segment (start 105.749 100.584) (end 105.7275 100.5625) (width 0.6) (layer F.Cu) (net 4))
 (segment (start 106.78 100.5625) (end 106.8015 100.584) (width 0.2) (layer F.Cu) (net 4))
 (segment (start 103 100.2) (end 105.365 100.2) (width 0.2) (layer F.Cu) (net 4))
 (segment (start 105.365 100.2) (end 105.7275 100.5625) (width 0.2) (layer F.Cu) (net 4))
 (segment (start 106.78 100.5625) (end 106.8015 100.584) (width 0.2) (layer F.Cu) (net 4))
 (segment (start 96.1 95.2) (end 96.1 101.8) (width 0.4) (layer B.Cu) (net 6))
 (segment (start 97.3 105.3) (end 97.85 104.75) (width 0.4) (layer F.Cu) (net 6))
 (via (at 97.3 105.3) (size 0.41) (drill 0.4) (layers F.Cu B.Cu) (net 6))
 (segment (start 97.3 103) (end 97.3 105.3) (width 0.4) (layer B.Cu) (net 6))
 (segment (start 96.1 101.8) (end 97.3 103) (width 0.4) (layer B.Cu) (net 6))
 (segment (start 97.85 104.75) (end 97.85 104.5) (width 0.4) (layer F.Cu) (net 6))
 (segment (start 97.8 103) (end 97.8 104.45) (width 0.2) (layer F.Cu) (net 6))
 (segment (start 97.8 104.45) (end 97.85 104.5) (width 0.2) (layer F.Cu) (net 6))
 (segment (start 103 95.35) (end 103 95.8) (width 0.4) (layer F.Cu) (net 6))
 (segment (start 95.65 95.65) (end 95.65 96.25) (width 0.4) (layer F.Cu) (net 6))
 (segment (start 96.1 95.2) (end 95.65 95.65) (width 0.4) (layer F.Cu) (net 6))
 (via (at 96.1 95.2) (size 0.41) (drill 0.4) (layers F.Cu B.Cu) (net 6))
 (segment (start 101.8 95.2) (end 96.1 95.2) (width 0.4) (layer B.Cu) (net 6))
 (segment (start 102.7 96.1) (end 101.8 95.2) (width 0.4) (layer B.Cu) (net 6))
 (via (at 102.7 96.1) (size 0.41) (drill 0.4) (layers F.Cu B.Cu) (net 6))
 (segment (start 103 95.8) (end 102.7 96.1) (width 0.4) (layer F.Cu) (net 6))
 (segment (start 103 97.8) (end 103 95.35) (width 0.2) (layer F.Cu) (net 6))
 (segment (start 97.8 97) (end 97.8 96.5) (width 0.2) (layer F.Cu) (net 6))
 (segment (start 97.8 96.5) (end 97.55 96.25) (width 0.2) (layer F.Cu) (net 6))
 (segment (start 97.55 96.25) (end 95.65 96.25) (width 0.2) (layer F.Cu) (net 6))
 (segment (start 98.4 94.95) (end 97.95 94.95) (width 0.2) (layer F.Cu) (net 9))
 (segment (start 96.3 92.5) (end 95.35 92.5) (width 0.2) (layer F.Cu) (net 9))
 (segment (start 96.9 93.1) (end 96.3 92.5) (width 0.2) (layer F.Cu) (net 9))
 (segment (start 96.9 93.9) (end 96.9 93.1) (width 0.2) (layer F.Cu) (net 9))
 (segment (start 97.95 94.95) (end 96.9 93.9) (width 0.2) (layer F.Cu) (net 9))
 (segment (start 98.6 97) (end 98.6 95.15) (width 0.2) (layer F.Cu) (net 9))
 (segment (start 98.6 95.15) (end 98.4 94.95) (width 0.2) (layer F.Cu) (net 9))
 (segment (start 94.45 92.5) (end 94.45 93.7) (width 0.2) (layer F.Cu) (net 12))
 (segment (start 94.45 93.7) (end 94.15 94) (width 0.2) (layer F.Cu) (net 12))
 (segment (start 97 97.8) (end 95.6 97.8) (width 0.2) (layer F.Cu) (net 5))
 (segment (start 95.6 97.8) (end 95.45 97.65) (width 0.2) (layer F.Cu) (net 5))
 (segment (start 95.6 97.8) (end 95.45 97.65) (width 0.2) (layer F.Cu) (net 5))
 (segment (start 103 99.4) (end 104.3 99.4) (width 0.2) (layer F.Cu) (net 7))
 (segment (start 105.55 98.15) (end 105.55 97.75) (width 0.2) (layer F.Cu) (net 7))
 (segment (start 104.3 99.4) (end 105.55 98.15) (width 0.2) (layer F.Cu) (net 7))
 (segment (start 105.55 97.75) (end 105.5 97.75) (width 0.2) (layer F.Cu) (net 7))
 (segment (start 103 99) (end 103.9 99) (width 0.2) (layer F.Cu) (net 8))
 (segment (start 105.1 96.7) (end 105.55 96.7) (width 0.2) (layer F.Cu) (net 8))
 (segment (start 104.9 96.9) (end 105.1 96.7) (width 0.2) (layer F.Cu) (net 8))
 (segment (start 104.9 98) (end 104.9 96.9) (width 0.2) (layer F.Cu) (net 8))
 (segment (start 103.9 99) (end 104.9 98) (width 0.2) (layer F.Cu) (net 8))
 (segment (start 98.2 97) (end 98.2 96.4) (width 0.2) (layer F.Cu) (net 13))
 (segment (start 96.3 94) (end 95.65 94) (width 0.2) (layer F.Cu) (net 13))
 (segment (start 96.5 94.2) (end 96.3 94) (width 0.2) (layer F.Cu) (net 13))
 (segment (start 96.5 94.7) (end 96.5 94.2) (width 0.2) (layer F.Cu) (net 13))
 (segment (start 98.2 96.4) (end 96.5 94.7) (width 0.2) (layer F.Cu) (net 13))
 (segment (start 95.65 94) (end 95.65 94.05) (width 0.2) (layer F.Cu) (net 13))
 (segment (start 95.7 94) (end 95.65 94) (width 0.2) (layer F.Cu) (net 13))
 (segment (start 91.5 95) (end 89.65 95) (width 0.2) (layer F.Cu) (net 10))
 (segment (start 97 98.2) (end 93.7 98.2) (width 0.2) (layer F.Cu) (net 10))
 (segment (start 93.1 95.8) (end 92.3 95) (width 0.2) (layer F.Cu) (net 10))
 (segment (start 93.1 97.6) (end 93.1 95.8) (width 0.2) (layer F.Cu) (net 10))
 (segment (start 93.7 98.2) (end 93.1 97.6) (width 0.2) (layer F.Cu) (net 10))
 (segment (start 92.3 95) (end 91.5 95) (width 0.2) (layer F.Cu) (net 10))
 (segment (start 91.5 97.5) (end 89.65 97.5) (width 0.2) (layer F.Cu) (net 11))
 (segment (start 97 98.6) (end 92.6 98.6) (width 0.2) (layer F.Cu) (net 11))
 (segment (start 92.6 98.6) (end 91.5 97.5) (width 0.2) (layer F.Cu) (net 11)))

